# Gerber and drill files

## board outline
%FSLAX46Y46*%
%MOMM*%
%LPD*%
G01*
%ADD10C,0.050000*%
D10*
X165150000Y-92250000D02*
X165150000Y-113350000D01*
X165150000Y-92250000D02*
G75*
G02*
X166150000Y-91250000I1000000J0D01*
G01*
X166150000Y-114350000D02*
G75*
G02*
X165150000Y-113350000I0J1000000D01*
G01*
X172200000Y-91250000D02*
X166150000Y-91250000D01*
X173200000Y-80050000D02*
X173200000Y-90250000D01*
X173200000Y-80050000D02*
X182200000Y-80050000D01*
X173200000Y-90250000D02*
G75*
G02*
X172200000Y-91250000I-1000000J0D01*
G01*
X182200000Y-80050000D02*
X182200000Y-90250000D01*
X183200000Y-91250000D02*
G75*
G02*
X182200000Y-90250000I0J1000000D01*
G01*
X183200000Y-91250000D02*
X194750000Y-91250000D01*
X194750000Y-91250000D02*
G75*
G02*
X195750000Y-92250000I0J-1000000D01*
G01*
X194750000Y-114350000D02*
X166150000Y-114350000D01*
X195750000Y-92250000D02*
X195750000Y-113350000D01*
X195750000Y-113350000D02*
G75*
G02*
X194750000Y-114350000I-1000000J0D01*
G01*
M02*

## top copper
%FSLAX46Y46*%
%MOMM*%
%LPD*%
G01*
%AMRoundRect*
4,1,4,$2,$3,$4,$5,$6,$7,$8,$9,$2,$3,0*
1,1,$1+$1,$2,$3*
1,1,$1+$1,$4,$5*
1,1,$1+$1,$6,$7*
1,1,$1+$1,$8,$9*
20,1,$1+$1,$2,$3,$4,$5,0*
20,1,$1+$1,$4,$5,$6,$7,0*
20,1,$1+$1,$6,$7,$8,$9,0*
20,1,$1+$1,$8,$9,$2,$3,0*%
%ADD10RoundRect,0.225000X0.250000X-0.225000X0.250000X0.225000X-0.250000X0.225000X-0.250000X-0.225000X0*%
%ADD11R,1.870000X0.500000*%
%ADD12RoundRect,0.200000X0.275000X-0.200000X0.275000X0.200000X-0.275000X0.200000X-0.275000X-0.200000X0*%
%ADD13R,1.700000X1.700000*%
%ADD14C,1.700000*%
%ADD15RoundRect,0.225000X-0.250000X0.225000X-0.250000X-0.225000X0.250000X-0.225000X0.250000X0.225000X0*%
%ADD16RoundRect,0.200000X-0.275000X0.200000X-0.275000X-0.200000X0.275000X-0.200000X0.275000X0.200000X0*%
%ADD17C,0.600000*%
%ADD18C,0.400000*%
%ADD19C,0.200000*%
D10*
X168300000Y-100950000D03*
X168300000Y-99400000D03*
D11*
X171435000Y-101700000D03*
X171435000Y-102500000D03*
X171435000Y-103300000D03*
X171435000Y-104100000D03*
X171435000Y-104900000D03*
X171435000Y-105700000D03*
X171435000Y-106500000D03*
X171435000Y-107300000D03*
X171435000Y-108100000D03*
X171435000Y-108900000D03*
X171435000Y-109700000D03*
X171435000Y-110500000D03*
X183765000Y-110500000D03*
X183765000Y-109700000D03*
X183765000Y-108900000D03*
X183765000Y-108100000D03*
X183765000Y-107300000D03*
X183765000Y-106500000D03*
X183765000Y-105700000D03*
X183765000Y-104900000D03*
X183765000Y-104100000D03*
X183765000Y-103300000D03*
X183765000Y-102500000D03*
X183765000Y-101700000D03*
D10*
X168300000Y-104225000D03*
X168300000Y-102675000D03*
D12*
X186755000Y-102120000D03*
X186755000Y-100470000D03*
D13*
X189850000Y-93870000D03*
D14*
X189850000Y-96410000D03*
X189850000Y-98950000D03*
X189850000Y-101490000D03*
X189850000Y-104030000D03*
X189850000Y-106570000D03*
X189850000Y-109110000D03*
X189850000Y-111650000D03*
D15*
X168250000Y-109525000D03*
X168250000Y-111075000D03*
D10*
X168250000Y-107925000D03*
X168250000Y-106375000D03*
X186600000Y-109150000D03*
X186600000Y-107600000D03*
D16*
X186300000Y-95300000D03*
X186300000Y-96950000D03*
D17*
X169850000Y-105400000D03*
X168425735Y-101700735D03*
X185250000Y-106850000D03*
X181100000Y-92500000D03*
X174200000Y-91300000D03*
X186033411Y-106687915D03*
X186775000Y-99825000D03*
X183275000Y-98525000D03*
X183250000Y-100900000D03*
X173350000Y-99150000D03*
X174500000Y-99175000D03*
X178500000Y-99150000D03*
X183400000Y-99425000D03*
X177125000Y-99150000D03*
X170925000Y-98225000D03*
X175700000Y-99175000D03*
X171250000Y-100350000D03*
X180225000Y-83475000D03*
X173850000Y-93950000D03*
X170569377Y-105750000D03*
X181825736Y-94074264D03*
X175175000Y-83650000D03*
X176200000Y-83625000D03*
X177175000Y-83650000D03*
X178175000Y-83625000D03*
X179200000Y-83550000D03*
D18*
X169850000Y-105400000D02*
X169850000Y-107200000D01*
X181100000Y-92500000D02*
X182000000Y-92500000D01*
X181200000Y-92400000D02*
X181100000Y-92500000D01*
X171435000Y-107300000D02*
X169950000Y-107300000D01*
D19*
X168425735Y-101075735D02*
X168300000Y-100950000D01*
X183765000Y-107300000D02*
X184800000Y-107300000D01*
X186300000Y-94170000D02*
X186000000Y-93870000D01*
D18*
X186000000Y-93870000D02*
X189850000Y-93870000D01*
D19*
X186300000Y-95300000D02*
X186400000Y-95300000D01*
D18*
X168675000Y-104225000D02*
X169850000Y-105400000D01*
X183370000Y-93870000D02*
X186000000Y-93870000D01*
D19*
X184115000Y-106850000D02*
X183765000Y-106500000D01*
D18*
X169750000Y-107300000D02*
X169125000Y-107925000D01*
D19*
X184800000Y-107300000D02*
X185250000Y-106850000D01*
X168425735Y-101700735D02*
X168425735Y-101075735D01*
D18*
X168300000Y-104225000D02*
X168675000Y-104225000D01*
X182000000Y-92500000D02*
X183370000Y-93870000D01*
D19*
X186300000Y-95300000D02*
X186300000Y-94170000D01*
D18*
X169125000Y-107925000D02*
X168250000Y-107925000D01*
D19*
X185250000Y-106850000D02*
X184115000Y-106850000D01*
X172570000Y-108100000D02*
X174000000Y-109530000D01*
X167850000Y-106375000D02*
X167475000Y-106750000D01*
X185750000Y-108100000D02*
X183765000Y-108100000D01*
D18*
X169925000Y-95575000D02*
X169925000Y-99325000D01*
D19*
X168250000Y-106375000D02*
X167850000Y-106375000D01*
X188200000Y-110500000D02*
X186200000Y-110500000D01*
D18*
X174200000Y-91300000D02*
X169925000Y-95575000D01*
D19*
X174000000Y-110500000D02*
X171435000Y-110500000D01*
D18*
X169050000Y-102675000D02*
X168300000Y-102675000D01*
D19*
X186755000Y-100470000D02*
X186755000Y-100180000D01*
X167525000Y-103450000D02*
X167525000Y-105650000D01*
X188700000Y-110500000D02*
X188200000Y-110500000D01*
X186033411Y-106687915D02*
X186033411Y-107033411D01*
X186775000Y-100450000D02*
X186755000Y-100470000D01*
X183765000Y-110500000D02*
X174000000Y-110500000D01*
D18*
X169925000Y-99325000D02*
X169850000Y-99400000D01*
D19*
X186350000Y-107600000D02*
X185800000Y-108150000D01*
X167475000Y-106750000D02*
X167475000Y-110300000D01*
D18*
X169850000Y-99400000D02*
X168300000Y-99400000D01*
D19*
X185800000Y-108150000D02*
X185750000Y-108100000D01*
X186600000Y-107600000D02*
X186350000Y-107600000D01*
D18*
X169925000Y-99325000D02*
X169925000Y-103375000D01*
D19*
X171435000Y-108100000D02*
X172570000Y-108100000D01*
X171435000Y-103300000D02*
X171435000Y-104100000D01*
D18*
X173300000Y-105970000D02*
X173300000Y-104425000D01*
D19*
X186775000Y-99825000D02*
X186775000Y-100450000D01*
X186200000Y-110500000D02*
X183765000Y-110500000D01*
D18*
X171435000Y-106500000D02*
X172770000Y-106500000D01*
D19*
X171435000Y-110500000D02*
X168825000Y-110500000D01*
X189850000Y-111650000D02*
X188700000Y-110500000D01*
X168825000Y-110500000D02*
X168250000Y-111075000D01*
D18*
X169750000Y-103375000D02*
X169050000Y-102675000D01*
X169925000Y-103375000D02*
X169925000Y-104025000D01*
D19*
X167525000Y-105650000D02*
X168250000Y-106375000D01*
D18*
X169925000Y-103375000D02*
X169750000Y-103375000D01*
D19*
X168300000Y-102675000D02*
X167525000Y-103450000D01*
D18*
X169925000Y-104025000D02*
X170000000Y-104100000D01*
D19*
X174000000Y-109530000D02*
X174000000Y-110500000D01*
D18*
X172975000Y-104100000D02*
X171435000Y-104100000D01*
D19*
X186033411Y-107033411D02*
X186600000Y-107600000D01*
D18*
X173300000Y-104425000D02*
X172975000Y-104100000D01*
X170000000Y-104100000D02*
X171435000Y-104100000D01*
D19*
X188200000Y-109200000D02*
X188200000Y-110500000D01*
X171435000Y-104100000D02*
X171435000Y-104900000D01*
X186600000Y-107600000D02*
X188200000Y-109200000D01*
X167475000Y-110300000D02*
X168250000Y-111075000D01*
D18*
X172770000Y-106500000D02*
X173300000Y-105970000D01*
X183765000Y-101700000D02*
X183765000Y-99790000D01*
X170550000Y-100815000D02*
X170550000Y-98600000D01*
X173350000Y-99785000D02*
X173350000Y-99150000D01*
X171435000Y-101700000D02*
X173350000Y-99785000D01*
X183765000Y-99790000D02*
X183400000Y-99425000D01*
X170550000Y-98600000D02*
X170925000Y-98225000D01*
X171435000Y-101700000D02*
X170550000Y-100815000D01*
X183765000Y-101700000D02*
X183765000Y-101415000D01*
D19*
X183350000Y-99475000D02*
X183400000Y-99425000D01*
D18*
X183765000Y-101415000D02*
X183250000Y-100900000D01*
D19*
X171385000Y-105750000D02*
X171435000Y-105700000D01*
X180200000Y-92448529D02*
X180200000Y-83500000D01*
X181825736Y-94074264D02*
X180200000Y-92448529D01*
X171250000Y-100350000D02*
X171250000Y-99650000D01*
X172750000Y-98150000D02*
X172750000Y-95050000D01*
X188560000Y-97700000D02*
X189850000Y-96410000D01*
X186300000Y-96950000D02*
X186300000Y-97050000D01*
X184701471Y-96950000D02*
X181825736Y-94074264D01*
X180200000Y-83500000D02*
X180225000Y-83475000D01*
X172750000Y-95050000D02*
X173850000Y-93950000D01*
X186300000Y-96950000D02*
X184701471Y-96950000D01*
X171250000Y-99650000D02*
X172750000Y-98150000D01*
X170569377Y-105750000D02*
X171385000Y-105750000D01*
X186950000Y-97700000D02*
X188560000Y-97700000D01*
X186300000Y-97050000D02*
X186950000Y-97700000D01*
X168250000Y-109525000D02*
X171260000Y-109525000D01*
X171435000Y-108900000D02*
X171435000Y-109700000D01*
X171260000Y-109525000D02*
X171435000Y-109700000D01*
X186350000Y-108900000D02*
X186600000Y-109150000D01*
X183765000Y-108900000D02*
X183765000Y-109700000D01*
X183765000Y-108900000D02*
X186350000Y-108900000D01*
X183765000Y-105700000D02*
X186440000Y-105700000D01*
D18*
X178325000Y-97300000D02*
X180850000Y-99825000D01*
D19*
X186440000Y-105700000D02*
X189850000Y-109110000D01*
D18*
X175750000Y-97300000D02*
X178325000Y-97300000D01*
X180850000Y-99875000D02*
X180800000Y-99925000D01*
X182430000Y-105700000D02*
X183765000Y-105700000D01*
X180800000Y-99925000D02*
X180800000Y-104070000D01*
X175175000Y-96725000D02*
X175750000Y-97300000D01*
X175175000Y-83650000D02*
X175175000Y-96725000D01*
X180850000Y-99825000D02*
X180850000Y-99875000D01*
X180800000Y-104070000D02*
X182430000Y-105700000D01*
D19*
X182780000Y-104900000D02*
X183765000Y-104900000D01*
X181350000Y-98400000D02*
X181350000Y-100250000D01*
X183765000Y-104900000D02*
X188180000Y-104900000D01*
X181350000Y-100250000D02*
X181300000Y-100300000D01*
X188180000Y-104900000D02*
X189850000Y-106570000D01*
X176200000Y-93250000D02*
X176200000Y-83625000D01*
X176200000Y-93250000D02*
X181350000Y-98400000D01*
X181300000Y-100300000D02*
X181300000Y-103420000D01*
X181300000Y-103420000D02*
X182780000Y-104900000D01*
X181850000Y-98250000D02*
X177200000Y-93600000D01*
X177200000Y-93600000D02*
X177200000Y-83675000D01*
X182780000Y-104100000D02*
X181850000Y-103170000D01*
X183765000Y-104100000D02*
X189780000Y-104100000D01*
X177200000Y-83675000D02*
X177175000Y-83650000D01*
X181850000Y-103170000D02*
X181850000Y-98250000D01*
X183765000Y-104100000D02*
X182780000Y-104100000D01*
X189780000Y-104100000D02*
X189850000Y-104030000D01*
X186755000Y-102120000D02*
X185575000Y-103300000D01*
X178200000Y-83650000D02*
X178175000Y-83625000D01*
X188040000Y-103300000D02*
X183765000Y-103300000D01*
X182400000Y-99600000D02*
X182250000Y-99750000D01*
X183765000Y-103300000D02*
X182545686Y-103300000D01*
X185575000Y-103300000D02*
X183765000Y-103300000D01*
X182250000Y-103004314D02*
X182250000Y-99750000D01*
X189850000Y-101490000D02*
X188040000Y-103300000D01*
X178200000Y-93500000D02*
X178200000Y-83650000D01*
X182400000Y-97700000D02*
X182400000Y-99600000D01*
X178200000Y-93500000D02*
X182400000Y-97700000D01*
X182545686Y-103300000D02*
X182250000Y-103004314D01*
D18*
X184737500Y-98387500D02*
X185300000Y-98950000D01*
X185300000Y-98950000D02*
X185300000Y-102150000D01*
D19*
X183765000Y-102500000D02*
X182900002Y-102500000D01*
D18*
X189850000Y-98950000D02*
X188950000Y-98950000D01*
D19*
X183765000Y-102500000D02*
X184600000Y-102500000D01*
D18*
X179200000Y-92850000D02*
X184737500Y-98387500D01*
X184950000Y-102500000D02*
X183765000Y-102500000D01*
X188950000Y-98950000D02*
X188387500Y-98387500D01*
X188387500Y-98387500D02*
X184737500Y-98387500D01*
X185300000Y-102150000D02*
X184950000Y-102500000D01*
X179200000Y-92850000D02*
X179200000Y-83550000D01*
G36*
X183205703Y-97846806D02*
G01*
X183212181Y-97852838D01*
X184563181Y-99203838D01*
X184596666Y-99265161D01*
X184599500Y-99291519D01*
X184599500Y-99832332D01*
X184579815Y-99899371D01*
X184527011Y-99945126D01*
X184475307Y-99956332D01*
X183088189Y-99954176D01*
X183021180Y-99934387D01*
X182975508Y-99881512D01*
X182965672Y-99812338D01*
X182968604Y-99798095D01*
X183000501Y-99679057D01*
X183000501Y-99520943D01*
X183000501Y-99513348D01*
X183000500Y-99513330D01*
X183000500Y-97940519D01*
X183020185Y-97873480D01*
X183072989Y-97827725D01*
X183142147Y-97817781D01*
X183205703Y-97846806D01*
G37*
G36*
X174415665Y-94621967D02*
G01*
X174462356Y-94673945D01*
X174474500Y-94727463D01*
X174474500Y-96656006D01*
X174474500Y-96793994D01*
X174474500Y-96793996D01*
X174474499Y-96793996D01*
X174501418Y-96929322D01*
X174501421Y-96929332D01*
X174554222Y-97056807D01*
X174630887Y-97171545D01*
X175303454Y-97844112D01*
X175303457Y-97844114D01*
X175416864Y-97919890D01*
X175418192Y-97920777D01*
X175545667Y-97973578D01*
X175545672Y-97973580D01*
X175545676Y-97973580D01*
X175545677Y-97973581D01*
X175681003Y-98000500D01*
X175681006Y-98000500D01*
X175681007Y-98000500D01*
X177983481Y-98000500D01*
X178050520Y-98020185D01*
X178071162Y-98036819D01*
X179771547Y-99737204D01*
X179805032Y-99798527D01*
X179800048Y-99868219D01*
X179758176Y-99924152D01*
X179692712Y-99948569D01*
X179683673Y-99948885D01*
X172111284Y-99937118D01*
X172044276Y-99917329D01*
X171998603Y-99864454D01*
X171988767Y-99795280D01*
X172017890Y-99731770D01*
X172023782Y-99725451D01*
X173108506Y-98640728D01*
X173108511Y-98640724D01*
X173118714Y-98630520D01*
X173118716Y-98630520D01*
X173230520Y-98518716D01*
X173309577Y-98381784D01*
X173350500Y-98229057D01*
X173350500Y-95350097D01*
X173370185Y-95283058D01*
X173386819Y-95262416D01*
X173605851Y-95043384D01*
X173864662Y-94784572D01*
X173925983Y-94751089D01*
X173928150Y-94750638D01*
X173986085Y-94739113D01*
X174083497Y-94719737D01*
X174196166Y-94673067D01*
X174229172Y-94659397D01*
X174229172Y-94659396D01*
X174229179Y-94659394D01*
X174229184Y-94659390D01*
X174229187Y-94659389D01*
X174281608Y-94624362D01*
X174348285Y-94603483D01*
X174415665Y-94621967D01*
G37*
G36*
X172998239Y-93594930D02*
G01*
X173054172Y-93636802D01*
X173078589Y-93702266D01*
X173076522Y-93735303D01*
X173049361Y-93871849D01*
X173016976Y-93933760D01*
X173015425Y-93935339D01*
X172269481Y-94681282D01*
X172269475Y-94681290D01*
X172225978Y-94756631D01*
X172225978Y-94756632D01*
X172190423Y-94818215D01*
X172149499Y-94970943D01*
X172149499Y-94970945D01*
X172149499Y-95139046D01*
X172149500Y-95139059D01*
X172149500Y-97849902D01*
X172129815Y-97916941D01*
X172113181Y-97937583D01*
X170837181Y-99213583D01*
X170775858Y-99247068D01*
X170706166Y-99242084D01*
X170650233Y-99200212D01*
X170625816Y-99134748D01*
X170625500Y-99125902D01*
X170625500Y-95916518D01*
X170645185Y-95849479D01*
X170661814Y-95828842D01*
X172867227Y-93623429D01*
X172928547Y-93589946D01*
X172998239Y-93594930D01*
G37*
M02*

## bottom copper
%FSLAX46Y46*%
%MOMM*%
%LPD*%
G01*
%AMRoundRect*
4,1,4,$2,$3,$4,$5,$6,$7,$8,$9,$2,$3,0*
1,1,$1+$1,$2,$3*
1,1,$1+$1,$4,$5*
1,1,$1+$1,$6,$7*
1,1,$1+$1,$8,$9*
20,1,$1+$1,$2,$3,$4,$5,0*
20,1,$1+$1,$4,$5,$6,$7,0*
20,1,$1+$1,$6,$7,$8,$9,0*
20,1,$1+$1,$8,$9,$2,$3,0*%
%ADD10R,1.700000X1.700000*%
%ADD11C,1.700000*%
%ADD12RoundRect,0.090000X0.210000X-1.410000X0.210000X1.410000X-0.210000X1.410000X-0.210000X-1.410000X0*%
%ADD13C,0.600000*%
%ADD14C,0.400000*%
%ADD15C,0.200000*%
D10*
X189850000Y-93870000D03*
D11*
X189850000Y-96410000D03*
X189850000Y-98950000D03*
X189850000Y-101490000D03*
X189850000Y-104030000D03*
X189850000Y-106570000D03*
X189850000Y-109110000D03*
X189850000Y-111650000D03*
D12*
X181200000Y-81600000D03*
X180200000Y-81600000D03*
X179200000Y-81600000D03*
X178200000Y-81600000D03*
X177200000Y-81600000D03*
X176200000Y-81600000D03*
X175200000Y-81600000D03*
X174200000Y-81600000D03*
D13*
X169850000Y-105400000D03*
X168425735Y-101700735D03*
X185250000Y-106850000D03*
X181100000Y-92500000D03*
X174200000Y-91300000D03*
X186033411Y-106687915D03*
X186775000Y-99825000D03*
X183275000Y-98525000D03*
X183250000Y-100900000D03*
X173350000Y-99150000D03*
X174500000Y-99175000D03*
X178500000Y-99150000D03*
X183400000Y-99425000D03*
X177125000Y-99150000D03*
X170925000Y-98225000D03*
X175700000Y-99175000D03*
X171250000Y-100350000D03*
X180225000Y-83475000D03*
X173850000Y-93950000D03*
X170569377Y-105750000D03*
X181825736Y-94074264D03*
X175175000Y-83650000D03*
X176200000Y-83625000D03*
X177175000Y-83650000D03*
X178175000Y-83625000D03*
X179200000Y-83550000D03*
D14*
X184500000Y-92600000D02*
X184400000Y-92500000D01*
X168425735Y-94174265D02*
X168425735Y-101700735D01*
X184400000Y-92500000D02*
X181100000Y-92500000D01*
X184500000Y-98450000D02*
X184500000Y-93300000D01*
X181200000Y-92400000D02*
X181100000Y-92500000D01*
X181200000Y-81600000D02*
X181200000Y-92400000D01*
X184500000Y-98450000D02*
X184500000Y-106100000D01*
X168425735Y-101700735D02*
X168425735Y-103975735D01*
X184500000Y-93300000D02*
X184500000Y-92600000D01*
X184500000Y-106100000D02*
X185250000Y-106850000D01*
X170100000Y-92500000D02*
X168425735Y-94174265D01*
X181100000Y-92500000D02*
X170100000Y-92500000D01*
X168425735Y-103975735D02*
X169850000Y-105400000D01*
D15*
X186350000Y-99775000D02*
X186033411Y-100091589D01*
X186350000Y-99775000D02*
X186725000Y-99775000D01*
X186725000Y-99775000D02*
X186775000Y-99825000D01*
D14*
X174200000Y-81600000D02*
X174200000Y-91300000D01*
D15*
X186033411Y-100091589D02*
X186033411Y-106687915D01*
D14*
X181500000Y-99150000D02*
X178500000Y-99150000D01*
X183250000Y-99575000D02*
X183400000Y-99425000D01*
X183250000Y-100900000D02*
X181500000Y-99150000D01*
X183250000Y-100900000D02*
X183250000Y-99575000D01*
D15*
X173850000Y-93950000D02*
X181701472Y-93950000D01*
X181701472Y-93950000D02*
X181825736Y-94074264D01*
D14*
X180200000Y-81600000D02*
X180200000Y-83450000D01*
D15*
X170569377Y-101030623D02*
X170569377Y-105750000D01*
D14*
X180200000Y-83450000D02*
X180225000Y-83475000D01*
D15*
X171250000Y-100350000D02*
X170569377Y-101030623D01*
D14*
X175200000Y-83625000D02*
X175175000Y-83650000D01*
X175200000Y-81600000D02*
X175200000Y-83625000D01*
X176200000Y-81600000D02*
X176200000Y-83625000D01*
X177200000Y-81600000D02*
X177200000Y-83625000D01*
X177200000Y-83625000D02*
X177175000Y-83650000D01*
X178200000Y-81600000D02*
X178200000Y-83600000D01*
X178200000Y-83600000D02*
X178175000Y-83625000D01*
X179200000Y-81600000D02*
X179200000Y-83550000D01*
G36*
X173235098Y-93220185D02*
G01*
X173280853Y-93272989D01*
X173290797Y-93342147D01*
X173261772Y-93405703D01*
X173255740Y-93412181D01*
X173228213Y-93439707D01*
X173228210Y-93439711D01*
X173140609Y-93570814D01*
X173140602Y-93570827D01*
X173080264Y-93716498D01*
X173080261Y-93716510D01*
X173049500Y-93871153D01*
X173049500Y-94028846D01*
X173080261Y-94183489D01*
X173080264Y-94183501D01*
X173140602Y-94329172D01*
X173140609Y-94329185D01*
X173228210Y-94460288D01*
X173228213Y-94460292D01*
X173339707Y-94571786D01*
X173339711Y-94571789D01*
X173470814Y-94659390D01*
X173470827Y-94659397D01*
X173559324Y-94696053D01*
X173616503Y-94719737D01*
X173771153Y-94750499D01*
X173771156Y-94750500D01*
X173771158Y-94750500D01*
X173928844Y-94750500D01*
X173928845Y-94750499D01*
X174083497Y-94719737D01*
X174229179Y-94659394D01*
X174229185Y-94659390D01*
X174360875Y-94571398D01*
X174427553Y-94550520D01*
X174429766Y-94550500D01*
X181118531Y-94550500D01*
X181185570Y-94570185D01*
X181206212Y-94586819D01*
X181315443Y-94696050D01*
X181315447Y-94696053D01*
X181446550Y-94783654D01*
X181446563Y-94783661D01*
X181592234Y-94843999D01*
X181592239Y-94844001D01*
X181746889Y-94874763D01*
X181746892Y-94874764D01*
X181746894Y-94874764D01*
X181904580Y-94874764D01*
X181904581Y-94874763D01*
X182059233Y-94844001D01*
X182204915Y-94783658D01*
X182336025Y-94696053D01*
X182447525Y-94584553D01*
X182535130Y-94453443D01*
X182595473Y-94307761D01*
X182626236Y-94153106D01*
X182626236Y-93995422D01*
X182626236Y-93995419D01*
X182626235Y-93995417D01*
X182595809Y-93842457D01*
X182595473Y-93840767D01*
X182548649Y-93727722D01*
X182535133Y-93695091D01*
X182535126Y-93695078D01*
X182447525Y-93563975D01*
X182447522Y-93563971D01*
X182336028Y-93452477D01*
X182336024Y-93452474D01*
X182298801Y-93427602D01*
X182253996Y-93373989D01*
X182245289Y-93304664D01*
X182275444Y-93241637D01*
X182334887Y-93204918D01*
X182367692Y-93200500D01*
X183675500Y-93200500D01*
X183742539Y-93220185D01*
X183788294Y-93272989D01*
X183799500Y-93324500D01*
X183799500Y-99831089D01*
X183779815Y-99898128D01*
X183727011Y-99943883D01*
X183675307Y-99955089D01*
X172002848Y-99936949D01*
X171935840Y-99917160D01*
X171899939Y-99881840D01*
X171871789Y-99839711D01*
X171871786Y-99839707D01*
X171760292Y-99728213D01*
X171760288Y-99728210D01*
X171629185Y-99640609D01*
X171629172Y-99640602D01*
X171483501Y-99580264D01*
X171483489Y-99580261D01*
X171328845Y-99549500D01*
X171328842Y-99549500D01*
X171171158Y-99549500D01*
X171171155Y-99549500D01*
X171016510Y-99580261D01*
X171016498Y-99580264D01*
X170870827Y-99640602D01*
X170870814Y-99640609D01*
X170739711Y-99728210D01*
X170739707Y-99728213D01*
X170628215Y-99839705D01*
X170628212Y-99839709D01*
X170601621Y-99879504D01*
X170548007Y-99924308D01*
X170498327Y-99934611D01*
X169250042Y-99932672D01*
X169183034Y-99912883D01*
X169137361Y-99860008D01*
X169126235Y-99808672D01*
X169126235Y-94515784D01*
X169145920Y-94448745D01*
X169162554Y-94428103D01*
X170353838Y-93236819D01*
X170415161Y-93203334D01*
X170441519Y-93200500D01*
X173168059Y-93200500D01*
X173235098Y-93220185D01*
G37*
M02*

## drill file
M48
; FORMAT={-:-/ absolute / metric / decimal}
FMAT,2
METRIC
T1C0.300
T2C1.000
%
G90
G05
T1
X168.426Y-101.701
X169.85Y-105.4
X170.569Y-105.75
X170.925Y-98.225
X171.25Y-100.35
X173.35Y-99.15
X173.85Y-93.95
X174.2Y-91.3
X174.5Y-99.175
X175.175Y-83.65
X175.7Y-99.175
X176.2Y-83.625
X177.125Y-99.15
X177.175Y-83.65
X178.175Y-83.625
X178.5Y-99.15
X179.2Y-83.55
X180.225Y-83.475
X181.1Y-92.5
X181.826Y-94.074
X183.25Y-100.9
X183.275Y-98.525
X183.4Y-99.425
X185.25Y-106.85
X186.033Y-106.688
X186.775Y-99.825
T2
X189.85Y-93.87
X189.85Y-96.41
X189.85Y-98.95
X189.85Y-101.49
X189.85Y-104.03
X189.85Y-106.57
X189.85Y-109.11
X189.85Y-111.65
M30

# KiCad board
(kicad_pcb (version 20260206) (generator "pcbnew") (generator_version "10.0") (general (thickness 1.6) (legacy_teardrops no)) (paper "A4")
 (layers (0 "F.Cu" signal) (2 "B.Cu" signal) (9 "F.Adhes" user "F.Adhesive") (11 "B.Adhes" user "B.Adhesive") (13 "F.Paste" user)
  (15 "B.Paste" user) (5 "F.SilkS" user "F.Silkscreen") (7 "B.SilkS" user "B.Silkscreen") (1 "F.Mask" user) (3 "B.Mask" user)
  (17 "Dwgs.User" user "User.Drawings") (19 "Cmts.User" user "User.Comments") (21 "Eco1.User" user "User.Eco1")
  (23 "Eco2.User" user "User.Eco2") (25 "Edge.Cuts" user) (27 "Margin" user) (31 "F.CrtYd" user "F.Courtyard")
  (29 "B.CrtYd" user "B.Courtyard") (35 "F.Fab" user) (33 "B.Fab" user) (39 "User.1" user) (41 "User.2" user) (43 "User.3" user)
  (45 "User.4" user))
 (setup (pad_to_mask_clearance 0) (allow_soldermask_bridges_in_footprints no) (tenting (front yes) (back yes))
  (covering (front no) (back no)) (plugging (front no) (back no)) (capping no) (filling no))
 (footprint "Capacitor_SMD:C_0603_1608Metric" (layer "F.Cu") (at 168.3 100.175 90)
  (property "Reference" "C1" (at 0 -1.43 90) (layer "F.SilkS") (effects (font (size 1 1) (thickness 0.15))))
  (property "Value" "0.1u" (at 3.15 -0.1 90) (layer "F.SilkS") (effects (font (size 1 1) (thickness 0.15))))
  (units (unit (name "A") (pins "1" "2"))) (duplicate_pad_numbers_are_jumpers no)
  (pad "1" smd roundrect (at -0.775 0 90) (size 0.9 0.95) (layers "F.Cu" "F.Mask" "F.Paste") (roundrect_rratio 0.25) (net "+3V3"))
  (pad "2" smd roundrect (at 0.775 0 90) (size 0.9 0.95) (layers "F.Cu" "F.Mask" "F.Paste") (roundrect_rratio 0.25) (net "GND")))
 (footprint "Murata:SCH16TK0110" (layer "F.Cu") (at 177.6 106.1)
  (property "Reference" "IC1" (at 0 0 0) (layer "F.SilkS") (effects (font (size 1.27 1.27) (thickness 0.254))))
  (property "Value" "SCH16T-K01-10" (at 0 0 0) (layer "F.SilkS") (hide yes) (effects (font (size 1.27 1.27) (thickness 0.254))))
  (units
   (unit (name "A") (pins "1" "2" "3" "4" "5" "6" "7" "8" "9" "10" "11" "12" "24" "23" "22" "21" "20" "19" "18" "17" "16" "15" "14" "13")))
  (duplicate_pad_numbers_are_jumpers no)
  (pad "1" smd rect (at -6.165 -4.4 90) (size 0.5 1.87) (layers "F.Cu" "F.Mask" "F.Paste") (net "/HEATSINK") (thermal_bridge_angle 45))
  (pad "2" smd rect (at -6.165 -3.6 90) (size 0.5 1.87) (layers "F.Cu" "F.Mask" "F.Paste") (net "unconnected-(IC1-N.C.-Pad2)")
   (thermal_bridge_angle 45))
  (pad "3" smd rect (at -6.165 -2.8 90) (size 0.5 1.87) (layers "F.Cu" "F.Mask" "F.Paste") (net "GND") (thermal_bridge_angle 45))
  (pad "4" smd rect (at -6.165 -2 90) (size 0.5 1.87) (layers "F.Cu" "F.Mask" "F.Paste") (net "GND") (thermal_bridge_angle 45))
  (pad "5" smd rect (at -6.165 -1.2 90) (size 0.5 1.87) (layers "F.Cu" "F.Mask" "F.Paste") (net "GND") (thermal_bridge_angle 45))
  (pad "6" smd rect (at -6.165 -0.4 90) (size 0.5 1.87) (layers "F.Cu" "F.Mask" "F.Paste") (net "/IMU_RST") (thermal_bridge_angle 45))
  (pad "7" smd rect (at -6.165 0.4 90) (size 0.5 1.87) (layers "F.Cu" "F.Mask" "F.Paste") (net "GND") (thermal_bridge_angle 45))
  (pad "8" smd rect (at -6.165 1.2 90) (size 0.5 1.87) (layers "F.Cu" "F.Mask" "F.Paste") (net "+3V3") (thermal_bridge_angle 45))
  (pad "9" smd rect (at -6.165 2 90) (size 0.5 1.87) (layers "F.Cu" "F.Mask" "F.Paste") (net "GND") (thermal_bridge_angle 45))
  (pad "10" smd rect (at -6.165 2.8 90) (size 0.5 1.87) (layers "F.Cu" "F.Mask" "F.Paste") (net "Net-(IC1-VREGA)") (thermal_bridge_angle 45))
  (pad "11" smd rect (at -6.165 3.6 90) (size 0.5 1.87) (layers "F.Cu" "F.Mask" "F.Paste") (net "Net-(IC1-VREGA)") (thermal_bridge_angle 45))
  (pad "12" smd rect (at -6.165 4.4 90) (size 0.5 1.87) (layers "F.Cu" "F.Mask" "F.Paste") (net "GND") (thermal_bridge_angle 45))
  (pad "13" smd rect (at 6.165 4.4 90) (size 0.5 1.87) (layers "F.Cu" "F.Mask" "F.Paste") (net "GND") (thermal_bridge_angle 45))
  (pad "14" smd rect (at 6.165 3.6 90) (size 0.5 1.87) (layers "F.Cu" "F.Mask" "F.Paste") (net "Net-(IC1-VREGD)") (thermal_bridge_angle 45))
  (pad "15" smd rect (at 6.165 2.8 90) (size 0.5 1.87) (layers "F.Cu" "F.Mask" "F.Paste") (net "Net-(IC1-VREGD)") (thermal_bridge_angle 45))
  (pad "16" smd rect (at 6.165 2 90) (size 0.5 1.87) (layers "F.Cu" "F.Mask" "F.Paste") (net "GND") (thermal_bridge_angle 45))
  (pad "17" smd rect (at 6.165 1.2 90) (size 0.5 1.87) (layers "F.Cu" "F.Mask" "F.Paste") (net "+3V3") (thermal_bridge_angle 45))
  (pad "18" smd rect (at 6.165 0.4 90) (size 0.5 1.87) (layers "F.Cu" "F.Mask" "F.Paste") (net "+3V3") (thermal_bridge_angle 45))
  (pad "19" smd rect (at 6.165 -0.4 90) (size 0.5 1.87) (layers "F.Cu" "F.Mask" "F.Paste") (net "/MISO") (thermal_bridge_angle 45))
  (pad "20" smd rect (at 6.165 -1.2 90) (size 0.5 1.87) (layers "F.Cu" "F.Mask" "F.Paste") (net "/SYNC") (thermal_bridge_angle 45))
  (pad "21" smd rect (at 6.165 -2 90) (size 0.5 1.87) (layers "F.Cu" "F.Mask" "F.Paste") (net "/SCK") (thermal_bridge_angle 45))
  (pad "22" smd rect (at 6.165 -2.8 90) (size 0.5 1.87) (layers "F.Cu" "F.Mask" "F.Paste") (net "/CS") (thermal_bridge_angle 45))
  (pad "23" smd rect (at 6.165 -3.6 90) (size 0.5 1.87) (layers "F.Cu" "F.Mask" "F.Paste") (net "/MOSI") (thermal_bridge_angle 45))
  (pad "24" smd rect (at 6.165 -4.4 90) (size 0.5 1.87) (layers "F.Cu" "F.Mask" "F.Paste") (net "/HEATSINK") (thermal_bridge_angle 45)))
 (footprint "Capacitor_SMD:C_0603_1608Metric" (layer "F.Cu") (at 168.3 103.45 90)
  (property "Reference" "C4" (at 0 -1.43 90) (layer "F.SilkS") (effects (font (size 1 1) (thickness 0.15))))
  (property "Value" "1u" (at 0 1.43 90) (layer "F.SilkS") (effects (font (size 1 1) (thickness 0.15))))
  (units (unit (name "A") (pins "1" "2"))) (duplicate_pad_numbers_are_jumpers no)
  (pad "1" smd roundrect (at -0.775 0 90) (size 0.9 0.95) (layers "F.Cu" "F.Mask" "F.Paste") (roundrect_rratio 0.25) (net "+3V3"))
  (pad "2" smd roundrect (at 0.775 0 90) (size 0.9 0.95) (layers "F.Cu" "F.Mask" "F.Paste") (roundrect_rratio 0.25) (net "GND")))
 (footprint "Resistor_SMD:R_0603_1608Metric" (layer "F.Cu") (at 186.755 101.295 90)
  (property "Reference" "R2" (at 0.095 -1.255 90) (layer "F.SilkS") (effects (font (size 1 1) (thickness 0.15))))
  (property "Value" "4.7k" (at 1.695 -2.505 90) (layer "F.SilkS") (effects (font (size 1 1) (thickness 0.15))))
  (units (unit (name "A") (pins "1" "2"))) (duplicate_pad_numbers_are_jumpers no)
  (pad "1" smd roundrect (at -0.825 0 90) (size 0.8 0.95) (layers "F.Cu" "F.Mask" "F.Paste") (roundrect_rratio 0.25) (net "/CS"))
  (pad "2" smd roundrect (at 0.825 0 90) (size 0.8 0.95) (layers "F.Cu" "F.Mask" "F.Paste") (roundrect_rratio 0.25) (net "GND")))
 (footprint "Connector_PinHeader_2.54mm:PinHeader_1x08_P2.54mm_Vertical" (layer "F.Cu") (at 189.85 93.87)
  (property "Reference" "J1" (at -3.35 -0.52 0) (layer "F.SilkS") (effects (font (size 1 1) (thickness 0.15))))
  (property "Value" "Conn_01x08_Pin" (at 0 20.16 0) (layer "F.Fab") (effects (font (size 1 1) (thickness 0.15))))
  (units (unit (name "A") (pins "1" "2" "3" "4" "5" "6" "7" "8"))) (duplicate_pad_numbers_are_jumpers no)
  (pad "1" thru_hole rect (at 0 0) (size 1.7 1.7) (drill 1) (layers "*.Cu" "*.Mask") (remove_unused_layers no) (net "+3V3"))
  (pad "2" thru_hole circle (at 0 2.54) (size 1.7 1.7) (drill 1) (layers "*.Cu" "*.Mask") (remove_unused_layers no) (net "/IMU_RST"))
  (pad "3" thru_hole circle (at 0 5.08) (size 1.7 1.7) (drill 1) (layers "*.Cu" "*.Mask") (remove_unused_layers no) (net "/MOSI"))
  (pad "4" thru_hole circle (at 0 7.62) (size 1.7 1.7) (drill 1) (layers "*.Cu" "*.Mask") (remove_unused_layers no) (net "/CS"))
  (pad "5" thru_hole circle (at 0 10.16) (size 1.7 1.7) (drill 1) (layers "*.Cu" "*.Mask") (remove_unused_layers no) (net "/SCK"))
  (pad "6" thru_hole circle (at 0 12.7) (size 1.7 1.7) (drill 1) (layers "*.Cu" "*.Mask") (remove_unused_layers no) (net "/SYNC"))
  (pad "7" thru_hole circle (at 0 15.24) (size 1.7 1.7) (drill 1) (layers "*.Cu" "*.Mask") (remove_unused_layers no) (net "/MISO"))
  (pad "8" thru_hole circle (at 0 17.78) (size 1.7 1.7) (drill 1) (layers "*.Cu" "*.Mask") (remove_unused_layers no) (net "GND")))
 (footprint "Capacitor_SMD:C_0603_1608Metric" (layer "F.Cu") (at 168.25 110.3 -90)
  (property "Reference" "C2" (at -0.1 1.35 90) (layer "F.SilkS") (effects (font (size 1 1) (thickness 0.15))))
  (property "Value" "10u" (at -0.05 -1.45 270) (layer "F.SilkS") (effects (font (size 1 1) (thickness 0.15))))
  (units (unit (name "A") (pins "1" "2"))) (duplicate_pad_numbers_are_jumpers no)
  (pad "1" smd roundrect (at -0.775 0 270) (size 0.9 0.95) (layers "F.Cu" "F.Mask" "F.Paste") (roundrect_rratio 0.25)
   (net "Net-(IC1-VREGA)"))
  (pad "2" smd roundrect (at 0.775 0 270) (size 0.9 0.95) (layers "F.Cu" "F.Mask" "F.Paste") (roundrect_rratio 0.25) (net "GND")))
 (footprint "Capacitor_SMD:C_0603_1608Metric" (layer "F.Cu") (at 168.25 107.15 90)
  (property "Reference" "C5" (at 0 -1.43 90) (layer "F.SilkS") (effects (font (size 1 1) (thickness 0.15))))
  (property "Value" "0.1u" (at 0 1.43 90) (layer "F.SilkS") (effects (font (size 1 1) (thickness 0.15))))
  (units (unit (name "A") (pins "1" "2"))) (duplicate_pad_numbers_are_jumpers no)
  (pad "1" smd roundrect (at -0.775 0 90) (size 0.9 0.95) (layers "F.Cu" "F.Mask" "F.Paste") (roundrect_rratio 0.25) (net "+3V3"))
  (pad "2" smd roundrect (at 0.775 0 90) (size 0.9 0.95) (layers "F.Cu" "F.Mask" "F.Paste") (roundrect_rratio 0.25) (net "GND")))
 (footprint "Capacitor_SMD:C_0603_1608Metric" (layer "F.Cu") (at 186.6 108.375 90)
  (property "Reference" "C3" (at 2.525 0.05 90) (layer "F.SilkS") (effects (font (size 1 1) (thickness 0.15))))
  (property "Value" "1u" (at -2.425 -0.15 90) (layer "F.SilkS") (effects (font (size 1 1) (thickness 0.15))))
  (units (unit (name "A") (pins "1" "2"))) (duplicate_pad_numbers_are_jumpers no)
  (pad "1" smd roundrect (at -0.775 0 90) (size 0.9 0.95) (layers "F.Cu" "F.Mask" "F.Paste") (roundrect_rratio 0.25) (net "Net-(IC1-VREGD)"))
  (pad "2" smd roundrect (at 0.775 0 90) (size 0.9 0.95) (layers "F.Cu" "F.Mask" "F.Paste") (roundrect_rratio 0.25) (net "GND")))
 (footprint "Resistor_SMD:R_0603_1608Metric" (layer "F.Cu") (at 186.3 96.125 -90)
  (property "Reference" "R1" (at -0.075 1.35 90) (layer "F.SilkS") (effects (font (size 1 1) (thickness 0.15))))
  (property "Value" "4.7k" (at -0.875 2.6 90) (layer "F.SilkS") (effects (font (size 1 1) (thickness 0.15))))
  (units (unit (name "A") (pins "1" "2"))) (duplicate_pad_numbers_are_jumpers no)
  (pad "1" smd roundrect (at -0.825 0 270) (size 0.8 0.95) (layers "F.Cu" "F.Mask" "F.Paste") (roundrect_rratio 0.25) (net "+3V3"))
  (pad "2" smd roundrect (at 0.825 0 270) (size 0.8 0.95) (layers "F.Cu" "F.Mask" "F.Paste") (roundrect_rratio 0.25) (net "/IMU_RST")))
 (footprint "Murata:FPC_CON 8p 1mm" (layer "B.Cu") (at 177.7 81.6 90)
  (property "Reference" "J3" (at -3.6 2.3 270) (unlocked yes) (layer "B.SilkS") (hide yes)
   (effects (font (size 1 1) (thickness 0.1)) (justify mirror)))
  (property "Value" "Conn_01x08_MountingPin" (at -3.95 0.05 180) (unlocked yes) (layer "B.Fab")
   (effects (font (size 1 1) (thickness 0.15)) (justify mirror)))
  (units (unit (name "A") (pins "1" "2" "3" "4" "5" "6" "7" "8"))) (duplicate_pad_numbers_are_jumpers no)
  (pad "1" smd roundrect (at 0 3.5 90) (size 3 0.6) (layers "B.Cu" "B.Mask" "B.Paste") (roundrect_rratio 0.15) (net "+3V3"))
  (pad "2" smd roundrect (at 0 2.5 90) (size 3 0.6) (layers "B.Cu" "B.Mask" "B.Paste") (roundrect_rratio 0.15) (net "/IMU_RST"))
  (pad "3" smd roundrect (at 0 1.5 90) (size 3 0.6) (layers "B.Cu" "B.Mask" "B.Paste") (roundrect_rratio 0.15) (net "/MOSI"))
  (pad "4" smd roundrect (at 0 0.5 90) (size 3 0.6) (layers "B.Cu" "B.Mask" "B.Paste") (roundrect_rratio 0.15) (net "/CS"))
  (pad "5" smd roundrect (at 0 -0.5 90) (size 3 0.6) (layers "B.Cu" "B.Mask" "B.Paste") (roundrect_rratio 0.15) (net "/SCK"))
  (pad "6" smd roundrect (at 0 -1.5 90) (size 3 0.6) (layers "B.Cu" "B.Mask" "B.Paste") (roundrect_rratio 0.15) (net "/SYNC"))
  (pad "7" smd roundrect (at 0 -2.5 90) (size 3 0.6) (layers "B.Cu" "B.Mask" "B.Paste") (roundrect_rratio 0.15) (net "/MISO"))
  (pad "8" smd roundrect (at 0 -3.5 90) (size 3 0.6) (layers "B.Cu" "B.Mask" "B.Paste") (roundrect_rratio 0.15) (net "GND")))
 (gr_line (start 165.15 92.25) (end 165.15 113.35) (stroke (width 0.05) (type default)) (layer "Edge.Cuts"))
 (gr_arc (start 165.15 92.25) (mid 165.442893 91.542893) (end 166.15 91.25) (stroke (width 0.05) (type default)) (layer "Edge.Cuts"))
 (gr_arc (start 166.15 114.35) (mid 165.442893 114.057107) (end 165.15 113.35) (stroke (width 0.05) (type default)) (layer "Edge.Cuts"))
 (gr_line (start 172.2 91.25) (end 166.15 91.25) (stroke (width 0.05) (type default)) (layer "Edge.Cuts"))
 (gr_line (start 173.2 80.05) (end 173.2 90.25) (stroke (width 0.05) (type default)) (layer "Edge.Cuts"))
 (gr_line (start 173.2 80.05) (end 182.2 80.05) (stroke (width 0.05) (type default)) (layer "Edge.Cuts"))
 (gr_arc (start 173.2 90.25) (mid 172.907107 90.957107) (end 172.2 91.25) (stroke (width 0.05) (type default)) (layer "Edge.Cuts"))
 (gr_line (start 182.2 80.05) (end 182.2 90.25) (stroke (width 0.05) (type default)) (layer "Edge.Cuts"))
 (gr_arc (start 183.2 91.25) (mid 182.492893 90.957107) (end 182.2 90.25) (stroke (width 0.05) (type default)) (layer "Edge.Cuts"))
 (gr_line (start 183.2 91.25) (end 194.75 91.25) (stroke (width 0.05) (type default)) (layer "Edge.Cuts"))
 (gr_arc (start 194.75 91.25) (mid 195.457107 91.542893) (end 195.75 92.25) (stroke (width 0.05) (type default)) (layer "Edge.Cuts"))
 (gr_line (start 194.75 114.35) (end 166.15 114.35) (stroke (width 0.05) (type default)) (layer "Edge.Cuts"))
 (gr_line (start 195.75 92.25) (end 195.75 113.35) (stroke (width 0.05) (type default)) (layer "Edge.Cuts"))
 (gr_arc (start 195.75 113.35) (mid 195.457107 114.057107) (end 194.75 114.35) (stroke (width 0.05) (type default)) (layer "Edge.Cuts"))
 (segment (start 169.85 105.4) (end 169.85 107.2) (width 0.4) (layer "F.Cu") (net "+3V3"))
 (segment (start 181.1 92.5) (end 182 92.5) (width 0.4) (layer "F.Cu") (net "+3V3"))
 (segment (start 181.2 92.4) (end 181.1 92.5) (width 0.4) (layer "F.Cu") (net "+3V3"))
 (segment (start 171.435 107.3) (end 169.95 107.3) (width 0.4) (layer "F.Cu") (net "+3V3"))
 (segment (start 168.425735 101.075735) (end 168.3 100.95) (width 0.2) (layer "F.Cu") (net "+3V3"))
 (segment (start 183.765 107.3) (end 184.8 107.3) (width 0.2) (layer "F.Cu") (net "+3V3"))
 (segment (start 186.3 94.17) (end 186 93.87) (width 0.2) (layer "F.Cu") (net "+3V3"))
 (segment (start 186 93.87) (end 189.85 93.87) (width 0.4) (layer "F.Cu") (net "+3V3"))
 (segment (start 186.3 95.3) (end 186.4 95.3) (width 0.2) (layer "F.Cu") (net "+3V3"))
 (segment (start 168.675 104.225) (end 169.85 105.4) (width 0.4) (layer "F.Cu") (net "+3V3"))
 (segment (start 183.37 93.87) (end 186 93.87) (width 0.4) (layer "F.Cu") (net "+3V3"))
 (segment (start 184.115 106.85) (end 183.765 106.5) (width 0.2) (layer "F.Cu") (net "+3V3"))
 (segment (start 169.75 107.3) (end 169.125 107.925) (width 0.4) (layer "F.Cu") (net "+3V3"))
 (segment (start 184.8 107.3) (end 185.25 106.85) (width 0.2) (layer "F.Cu") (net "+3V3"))
 (segment (start 168.425735 101.700735) (end 168.425735 101.075735) (width 0.2) (layer "F.Cu") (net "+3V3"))
 (segment (start 168.3 104.225) (end 168.675 104.225) (width 0.4) (layer "F.Cu") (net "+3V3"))
 (segment (start 182 92.5) (end 183.37 93.87) (width 0.4) (layer "F.Cu") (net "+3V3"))
 (segment (start 186.3 95.3) (end 186.3 94.17) (width 0.2) (layer "F.Cu") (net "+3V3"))
 (segment (start 169.125 107.925) (end 168.25 107.925) (width 0.4) (layer "F.Cu") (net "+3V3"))
 (segment (start 185.25 106.85) (end 184.115 106.85) (width 0.2) (layer "F.Cu") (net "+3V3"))
 (via (at 169.85 105.4) (size 0.6) (drill 0.3) (layers "F.Cu" "B.Cu") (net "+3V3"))
 (via (at 168.425735 101.700735) (size 0.6) (drill 0.3) (layers "F.Cu" "B.Cu") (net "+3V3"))
 (via (at 185.25 106.85) (size 0.6) (drill 0.3) (layers "F.Cu" "B.Cu") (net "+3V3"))
 (via (at 181.1 92.5) (size 0.6) (drill 0.3) (layers "F.Cu" "B.Cu") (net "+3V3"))
 (segment (start 184.5 92.6) (end 184.4 92.5) (width 0.4) (layer "B.Cu") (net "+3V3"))
 (segment (start 168.425735 94.174265) (end 168.425735 101.700735) (width 0.4) (layer "B.Cu") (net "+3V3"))
 (segment (start 184.4 92.5) (end 181.1 92.5) (width 0.4) (layer "B.Cu") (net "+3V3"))
 (segment (start 184.5 98.45) (end 184.5 93.3) (width 0.4) (layer "B.Cu") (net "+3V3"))
 (segment (start 181.2 92.4) (end 181.1 92.5) (width 0.4) (layer "B.Cu") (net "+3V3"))
 (segment (start 181.2 81.6) (end 181.2 92.4) (width 0.4) (layer "B.Cu") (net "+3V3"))
 (segment (start 184.5 98.45) (end 184.5 106.1) (width 0.4) (layer "B.Cu") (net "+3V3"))
 (segment (start 168.425735 101.700735) (end 168.425735 103.975735) (width 0.4) (layer "B.Cu") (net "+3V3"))
 (segment (start 184.5 93.3) (end 184.5 92.6) (width 0.4) (layer "B.Cu") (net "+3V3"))
 (segment (start 184.5 106.1) (end 185.25 106.85) (width 0.4) (layer "B.Cu") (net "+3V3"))
 (segment (start 170.1 92.5) (end 168.425735 94.174265) (width 0.4) (layer "B.Cu") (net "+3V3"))
 (segment (start 181.1 92.5) (end 170.1 92.5) (width 0.4) (layer "B.Cu") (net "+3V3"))
 (segment (start 168.425735 103.975735) (end 169.85 105.4) (width 0.4) (layer "B.Cu") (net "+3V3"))
 (segment (start 172.57 108.1) (end 174 109.53) (width 0.2) (layer "F.Cu") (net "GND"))
 (segment (start 167.85 106.375) (end 167.475 106.75) (width 0.2) (layer "F.Cu") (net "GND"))
 (segment (start 185.75 108.1) (end 183.765 108.1) (width 0.2) (layer "F.Cu") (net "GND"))
 (segment (start 169.925 95.575) (end 169.925 99.325) (width 0.4) (layer "F.Cu") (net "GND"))
 (segment (start 168.25 106.375) (end 167.85 106.375) (width 0.2) (layer "F.Cu") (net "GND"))
 (segment (start 188.2 110.5) (end 186.2 110.5) (width 0.2) (layer "F.Cu") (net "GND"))
 (segment (start 174.2 91.3) (end 169.925 95.575) (width 0.4) (layer "F.Cu") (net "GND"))
 (segment (start 174 110.5) (end 171.435 110.5) (width 0.2) (layer "F.Cu") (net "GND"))
 (segment (start 169.05 102.675) (end 168.3 102.675) (width 0.4) (layer "F.Cu") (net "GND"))
 (segment (start 186.755 100.47) (end 186.755 100.18) (width 0.2) (layer "F.Cu") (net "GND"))
 (segment (start 167.525 103.45) (end 167.525 105.65) (width 0.2) (layer "F.Cu") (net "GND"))
 (segment (start 188.7 110.5) (end 188.2 110.5) (width 0.2) (layer "F.Cu") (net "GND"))
 (segment (start 186.033411 106.687915) (end 186.033411 107.033411) (width 0.2) (layer "F.Cu") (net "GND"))
 (segment (start 186.775 100.45) (end 186.755 100.47) (width 0.2) (layer "F.Cu") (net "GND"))
 (segment (start 183.765 110.5) (end 174 110.5) (width 0.2) (layer "F.Cu") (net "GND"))
 (segment (start 169.925 99.325) (end 169.85 99.4) (width 0.4) (layer "F.Cu") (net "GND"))
 (segment (start 186.35 107.6) (end 185.8 108.15) (width 0.2) (layer "F.Cu") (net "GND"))
 (segment (start 167.475 106.75) (end 167.475 110.3) (width 0.2) (layer "F.Cu") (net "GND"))
 (segment (start 169.85 99.4) (end 168.3 99.4) (width 0.4) (layer "F.Cu") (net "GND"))
 (segment (start 185.8 108.15) (end 185.75 108.1) (width 0.2) (layer "F.Cu") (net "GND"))
 (segment (start 186.6 107.6) (end 186.35 107.6) (width 0.2) (layer "F.Cu") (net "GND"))
 (segment (start 169.925 99.325) (end 169.925 103.375) (width 0.4) (layer "F.Cu") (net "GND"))
 (segment (start 171.435 108.1) (end 172.57 108.1) (width 0.2) (layer "F.Cu") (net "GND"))
 (segment (start 171.435 103.3) (end 171.435 104.1) (width 0.2) (layer "F.Cu") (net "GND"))
 (segment (start 173.3 105.97) (end 173.3 104.425) (width 0.4) (layer "F.Cu") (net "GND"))
 (segment (start 186.775 99.825) (end 186.775 100.45) (width 0.2) (layer "F.Cu") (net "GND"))
 (segment (start 186.2 110.5) (end 183.765 110.5) (width 0.2) (layer "F.Cu") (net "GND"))
 (segment (start 171.435 106.5) (end 172.77 106.5) (width 0.4) (layer "F.Cu") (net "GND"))
 (segment (start 171.435 110.5) (end 168.825 110.5) (width 0.2) (layer "F.Cu") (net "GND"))
 (segment (start 189.85 111.65) (end 188.7 110.5) (width 0.2) (layer "F.Cu") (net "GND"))
 (segment (start 168.825 110.5) (end 168.25 111.075) (width 0.2) (layer "F.Cu") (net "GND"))
 (segment (start 169.75 103.375) (end 169.05 102.675) (width 0.4) (layer "F.Cu") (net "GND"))
 (segment (start 169.925 103.375) (end 169.925 104.025) (width 0.4) (layer "F.Cu") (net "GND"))
 (segment (start 167.525 105.65) (end 168.25 106.375) (width 0.2) (layer "F.Cu") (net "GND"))
 (segment (start 169.925 103.375) (end 169.75 103.375) (width 0.4) (layer "F.Cu") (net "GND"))
 (segment (start 168.3 102.675) (end 167.525 103.45) (width 0.2) (layer "F.Cu") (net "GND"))
 (segment (start 169.925 104.025) (end 170 104.1) (width 0.4) (layer "F.Cu") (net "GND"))
 (segment (start 174 109.53) (end 174 110.5) (width 0.2) (layer "F.Cu") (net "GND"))
 (segment (start 172.975 104.1) (end 171.435 104.1) (width 0.4) (layer "F.Cu") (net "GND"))
 (segment (start 186.033411 107.033411) (end 186.6 107.6) (width 0.2) (layer "F.Cu") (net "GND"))
 (segment (start 173.3 104.425) (end 172.975 104.1) (width 0.4) (layer "F.Cu") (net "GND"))
 (segment (start 170 104.1) (end 171.435 104.1) (width 0.4) (layer "F.Cu") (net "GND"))
 (segment (start 188.2 109.2) (end 188.2 110.5) (width 0.2) (layer "F.Cu") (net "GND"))
 (segment (start 171.435 104.1) (end 171.435 104.9) (width 0.2) (layer "F.Cu") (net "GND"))
 (segment (start 186.6 107.6) (end 188.2 109.2) (width 0.2) (layer "F.Cu") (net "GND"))
 (segment (start 167.475 110.3) (end 168.25 111.075) (width 0.2) (layer "F.Cu") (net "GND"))
 (segment (start 172.77 106.5) (end 173.3 105.97) (width 0.4) (layer "F.Cu") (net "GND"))
 (via (at 174.2 91.3) (size 0.6) (drill 0.3) (layers "F.Cu" "B.Cu") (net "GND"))
 (via (at 186.033411 106.687915) (size 0.6) (drill 0.3) (layers "F.Cu" "B.Cu") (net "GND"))
 (via (at 186.775 99.825) (size 0.6) (drill 0.3) (layers "F.Cu" "B.Cu") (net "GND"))
 (segment (start 186.35 99.775) (end 186.033411 100.091589) (width 0.2) (layer "B.Cu") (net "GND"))
 (segment (start 186.35 99.775) (end 186.725 99.775) (width 0.2) (layer "B.Cu") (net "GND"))
 (segment (start 186.725 99.775) (end 186.775 99.825) (width 0.2) (layer "B.Cu") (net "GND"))
 (segment (start 174.2 81.6) (end 174.2 91.3) (width 0.4) (layer "B.Cu") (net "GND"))
 (segment (start 186.033411 100.091589) (end 186.033411 106.687915) (width 0.2) (layer "B.Cu") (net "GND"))
 (segment (start 183.765 101.7) (end 183.765 99.79) (width 0.4) (layer "F.Cu") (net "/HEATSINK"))
 (segment (start 170.55 100.815) (end 170.55 98.6) (width 0.4) (layer "F.Cu") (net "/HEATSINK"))
 (segment (start 173.35 99.785) (end 173.35 99.15) (width 0.4) (layer "F.Cu") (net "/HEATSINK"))
 (segment (start 171.435 101.7) (end 173.35 99.785) (width 0.4) (layer "F.Cu") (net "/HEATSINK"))
 (segment (start 183.765 99.79) (end 183.4 99.425) (width 0.4) (layer "F.Cu") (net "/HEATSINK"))
 (segment (start 170.55 98.6) (end 170.925 98.225) (width 0.4) (layer "F.Cu") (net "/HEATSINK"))
 (segment (start 171.435 101.7) (end 170.55 100.815) (width 0.4) (layer "F.Cu") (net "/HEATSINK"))
 (segment (start 183.765 101.7) (end 183.765 101.415) (width 0.4) (layer "F.Cu") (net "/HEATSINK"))
 (segment (start 183.35 99.475) (end 183.4 99.425) (width 0.2) (layer "F.Cu") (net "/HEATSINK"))
 (segment (start 183.765 101.415) (end 183.25 100.9) (width 0.4) (layer "F.Cu") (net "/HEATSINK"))
 (via (at 183.275 98.525) (size 0.6) (drill 0.3) (layers "F.Cu" "B.Cu") (free yes) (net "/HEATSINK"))
 (via (at 183.25 100.9) (size 0.6) (drill 0.3) (layers "F.Cu" "B.Cu") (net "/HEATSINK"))
 (via (at 173.35 99.15) (size 0.6) (drill 0.3) (layers "F.Cu" "B.Cu") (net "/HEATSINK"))
 (via (at 174.5 99.175) (size 0.6) (drill 0.3) (layers "F.Cu" "B.Cu") (free yes) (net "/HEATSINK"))
 (via (at 178.5 99.15) (size 0.6) (drill 0.3) (layers "F.Cu" "B.Cu") (free yes) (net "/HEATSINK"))
 (via (at 183.4 99.425) (size 0.6) (drill 0.3) (layers "F.Cu" "B.Cu") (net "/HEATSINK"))
 (via (at 177.125 99.15) (size 0.6) (drill 0.3) (layers "F.Cu" "B.Cu") (free yes) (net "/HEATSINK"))
 (via (at 170.925 98.225) (size 0.6) (drill 0.3) (layers "F.Cu" "B.Cu") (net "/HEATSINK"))
 (via (at 175.7 99.175) (size 0.6) (drill 0.3) (layers "F.Cu" "B.Cu") (free yes) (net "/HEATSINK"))
 (segment (start 181.5 99.15) (end 178.5 99.15) (width 0.4) (layer "B.Cu") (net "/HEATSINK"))
 (segment (start 183.25 99.575) (end 183.4 99.425) (width 0.4) (layer "B.Cu") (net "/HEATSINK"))
 (segment (start 183.25 100.9) (end 181.5 99.15) (width 0.4) (layer "B.Cu") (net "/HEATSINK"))
 (segment (start 183.25 100.9) (end 183.25 99.575) (width 0.4) (layer "B.Cu") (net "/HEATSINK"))
 (segment (start 171.385 105.75) (end 171.435 105.7) (width 0.2) (layer "F.Cu") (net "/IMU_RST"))
 (segment (start 180.2 92.448529) (end 180.2 83.5) (width 0.2) (layer "F.Cu") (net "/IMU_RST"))
 (segment (start 181.825736 94.074264) (end 180.2 92.448529) (width 0.2) (layer "F.Cu") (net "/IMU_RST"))
 (segment (start 171.25 100.35) (end 171.25 99.65) (width 0.2) (layer "F.Cu") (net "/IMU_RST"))
 (segment (start 172.75 98.15) (end 172.75 95.05) (width 0.2) (layer "F.Cu") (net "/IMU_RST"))
 (segment (start 188.56 97.7) (end 189.85 96.41) (width 0.2) (layer "F.Cu") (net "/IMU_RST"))
 (segment (start 186.3 96.95) (end 186.3 97.05) (width 0.2) (layer "F.Cu") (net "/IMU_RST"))
 (segment (start 184.701471 96.95) (end 181.825736 94.074264) (width 0.2) (layer "F.Cu") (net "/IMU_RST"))
 (segment (start 180.2 83.5) (end 180.225 83.475) (width 0.2) (layer "F.Cu") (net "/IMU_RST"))
 (segment (start 172.75 95.05) (end 173.85 93.95) (width 0.2) (layer "F.Cu") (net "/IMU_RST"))
 (segment (start 186.3 96.95) (end 184.701471 96.95) (width 0.2) (layer "F.Cu") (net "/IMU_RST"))
 (segment (start 171.25 99.65) (end 172.75 98.15) (width 0.2) (layer "F.Cu") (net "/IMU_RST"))
 (segment (start 170.569377 105.75) (end 171.385 105.75) (width 0.2) (layer "F.Cu") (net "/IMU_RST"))
 (segment (start 186.95 97.7) (end 188.56 97.7) (width 0.2) (layer "F.Cu") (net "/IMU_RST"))
 (segment (start 186.3 97.05) (end 186.95 97.7) (width 0.2) (layer "F.Cu") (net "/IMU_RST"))
 (via (at 171.25 100.35) (size 0.6) (drill 0.3) (layers "F.Cu" "B.Cu") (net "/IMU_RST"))
 (via (at 180.225 83.475) (size 0.6) (drill 0.3) (layers "F.Cu" "B.Cu") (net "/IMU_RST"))
 (via (at 173.85 93.95) (size 0.6) (drill 0.3) (layers "F.Cu" "B.Cu") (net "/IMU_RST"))
 (via (at 170.569377 105.75) (size 0.6) (drill 0.3) (layers "F.Cu" "B.Cu") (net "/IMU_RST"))
 (via (at 181.825736 94.074264) (size 0.6) (drill 0.3) (layers "F.Cu" "B.Cu") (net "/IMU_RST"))
 (segment (start 173.85 93.95) (end 181.701472 93.95) (width 0.2) (layer "B.Cu") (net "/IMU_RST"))
 (segment (start 181.701472 93.95) (end 181.825736 94.074264) (width 0.2) (layer "B.Cu") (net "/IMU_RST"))
 (segment (start 180.2 81.6) (end 180.2 83.45) (width 0.4) (layer "B.Cu") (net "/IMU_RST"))
 (segment (start 170.569377 101.030623) (end 170.569377 105.75) (width 0.2) (layer "B.Cu") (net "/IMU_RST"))
 (segment (start 180.2 83.45) (end 180.225 83.475) (width 0.4) (layer "B.Cu") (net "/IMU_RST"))
 (segment (start 171.25 100.35) (end 170.569377 101.030623) (width 0.2) (layer "B.Cu") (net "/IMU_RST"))
 (segment (start 168.25 109.525) (end 171.26 109.525) (width 0.2) (layer "F.Cu") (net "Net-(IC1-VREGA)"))
 (segment (start 171.435 108.9) (end 171.435 109.7) (width 0.2) (layer "F.Cu") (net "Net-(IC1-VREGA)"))
 (segment (start 171.26 109.525) (end 171.435 109.7) (width 0.2) (layer "F.Cu") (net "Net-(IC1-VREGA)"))
 (segment (start 186.35 108.9) (end 186.6 109.15) (width 0.2) (layer "F.Cu") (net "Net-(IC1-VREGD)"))
 (segment (start 183.765 108.9) (end 183.765 109.7) (width 0.2) (layer "F.Cu") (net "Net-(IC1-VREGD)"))
 (segment (start 183.765 108.9) (end 186.35 108.9) (width 0.2) (layer "F.Cu") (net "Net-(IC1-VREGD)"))
 (segment (start 183.765 105.7) (end 186.44 105.7) (width 0.2) (layer "F.Cu") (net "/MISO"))
 (segment (start 178.325 97.3) (end 180.85 99.825) (width 0.4) (layer "F.Cu") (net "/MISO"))
 (segment (start 186.44 105.7) (end 189.85 109.11) (width 0.2) (layer "F.Cu") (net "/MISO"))
 (segment (start 175.75 97.3) (end 178.325 97.3) (width 0.4) (layer "F.Cu") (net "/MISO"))
 (segment (start 180.85 99.875) (end 180.8 99.925) (width 0.4) (layer "F.Cu") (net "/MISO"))
 (segment (start 182.43 105.7) (end 183.765 105.7) (width 0.4) (layer "F.Cu") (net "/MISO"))
 (segment (start 180.8 99.925) (end 180.8 104.07) (width 0.4) (layer "F.Cu") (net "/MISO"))
 (segment (start 175.175 96.725) (end 175.75 97.3) (width 0.4) (layer "F.Cu") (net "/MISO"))
 (segment (start 175.175 83.65) (end 175.175 96.725) (width 0.4) (layer "F.Cu") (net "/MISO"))
 (segment (start 180.85 99.825) (end 180.85 99.875) (width 0.4) (layer "F.Cu") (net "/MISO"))
 (segment (start 180.8 104.07) (end 182.43 105.7) (width 0.4) (layer "F.Cu") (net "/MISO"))
 (via (at 175.175 83.65) (size 0.6) (drill 0.3) (layers "F.Cu" "B.Cu") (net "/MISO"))
 (segment (start 175.2 83.625) (end 175.175 83.65) (width 0.4) (layer "B.Cu") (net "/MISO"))
 (segment (start 175.2 81.6) (end 175.2 83.625) (width 0.4) (layer "B.Cu") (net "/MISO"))
 (segment (start 182.78 104.9) (end 183.765 104.9) (width 0.2) (layer "F.Cu") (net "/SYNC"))
 (segment (start 181.35 98.4) (end 181.35 100.25) (width 0.2) (layer "F.Cu") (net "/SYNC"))
 (segment (start 183.765 104.9) (end 188.18 104.9) (width 0.2) (layer "F.Cu") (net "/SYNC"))
 (segment (start 181.35 100.25) (end 181.3 100.3) (width 0.2) (layer "F.Cu") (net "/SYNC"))
 (segment (start 188.18 104.9) (end 189.85 106.57) (width 0.2) (layer "F.Cu") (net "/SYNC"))
 (segment (start 176.2 93.25) (end 176.2 83.625) (width 0.2) (layer "F.Cu") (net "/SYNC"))
 (segment (start 176.2 93.25) (end 181.35 98.4) (width 0.2) (layer "F.Cu") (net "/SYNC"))
 (segment (start 181.3 100.3) (end 181.3 103.42) (width 0.2) (layer "F.Cu") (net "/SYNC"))
 (segment (start 181.3 103.42) (end 182.78 104.9) (width 0.2) (layer "F.Cu") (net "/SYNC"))
 (via (at 176.2 83.625) (size 0.6) (drill 0.3) (layers "F.Cu" "B.Cu") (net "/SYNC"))
 (segment (start 176.2 81.6) (end 176.2 83.625) (width 0.4) (layer "B.Cu") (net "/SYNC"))
 (segment (start 181.85 98.25) (end 177.2 93.6) (width 0.2) (layer "F.Cu") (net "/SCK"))
 (segment (start 177.2 93.6) (end 177.2 83.675) (width 0.2) (layer "F.Cu") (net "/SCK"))
 (segment (start 182.78 104.1) (end 181.85 103.17) (width 0.2) (layer "F.Cu") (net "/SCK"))
 (segment (start 183.765 104.1) (end 189.78 104.1) (width 0.2) (layer "F.Cu") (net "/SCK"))
 (segment (start 177.2 83.675) (end 177.175 83.65) (width 0.2) (layer "F.Cu") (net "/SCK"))
 (segment (start 181.85 103.17) (end 181.85 98.25) (width 0.2) (layer "F.Cu") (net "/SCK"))
 (segment (start 183.765 104.1) (end 182.78 104.1) (width 0.2) (layer "F.Cu") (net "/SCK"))
 (segment (start 189.78 104.1) (end 189.85 104.03) (width 0.2) (layer "F.Cu") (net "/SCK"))
 (via (at 177.175 83.65) (size 0.6) (drill 0.3) (layers "F.Cu" "B.Cu") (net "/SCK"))
 (segment (start 177.2 81.6) (end 177.2 83.625) (width 0.4) (layer "B.Cu") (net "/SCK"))
 (segment (start 177.2 83.625) (end 177.175 83.65) (width 0.4) (layer "B.Cu") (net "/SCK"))
 (segment (start 186.755 102.12) (end 185.575 103.3) (width 0.2) (layer "F.Cu") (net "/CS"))
 (segment (start 178.2 83.65) (end 178.175 83.625) (width 0.2) (layer "F.Cu") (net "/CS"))
 (segment (start 188.04 103.3) (end 183.765 103.3) (width 0.2) (layer "F.Cu") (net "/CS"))
 (segment (start 182.4 99.6) (end 182.25 99.75) (width 0.2) (layer "F.Cu") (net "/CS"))
 (segment (start 183.765 103.3) (end 182.545686 103.3) (width 0.2) (layer "F.Cu") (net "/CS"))
 (segment (start 185.575 103.3) (end 183.765 103.3) (width 0.2) (layer "F.Cu") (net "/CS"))
 (segment (start 182.25 103.004314) (end 182.25 99.75) (width 0.2) (layer "F.Cu") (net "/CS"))
 (segment (start 189.85 101.49) (end 188.04 103.3) (width 0.2) (layer "F.Cu") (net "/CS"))
 (segment (start 178.2 93.5) (end 178.2 83.65) (width 0.2) (layer "F.Cu") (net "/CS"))
 (segment (start 182.4 97.7) (end 182.4 99.6) (width 0.2) (layer "F.Cu") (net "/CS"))
 (segment (start 178.2 93.5) (end 182.4 97.7) (width 0.2) (layer "F.Cu") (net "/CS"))
 (segment (start 182.545686 103.3) (end 182.25 103.004314) (width 0.2) (layer "F.Cu") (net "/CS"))
 (via (at 178.175 83.625) (size 0.6) (drill 0.3) (layers "F.Cu" "B.Cu") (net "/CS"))
 (segment (start 178.2 81.6) (end 178.2 83.6) (width 0.4) (layer "B.Cu") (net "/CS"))
 (segment (start 178.2 83.6) (end 178.175 83.625) (width 0.4) (layer "B.Cu") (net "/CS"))
 (segment (start 184.7375 98.3875) (end 185.3 98.95) (width 0.4) (layer "F.Cu") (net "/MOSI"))
 (segment (start 185.3 98.95) (end 185.3 102.15) (width 0.4) (layer "F.Cu") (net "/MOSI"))
 (segment (start 183.765 102.5) (end 182.900002 102.5) (width 0.2) (layer "F.Cu") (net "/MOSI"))
 (segment (start 189.85 98.95) (end 188.95 98.95) (width 0.4) (layer "F.Cu") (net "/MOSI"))
 (segment (start 183.765 102.5) (end 184.6 102.5) (width 0.2) (layer "F.Cu") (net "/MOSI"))
 (segment (start 179.2 92.85) (end 184.7375 98.3875) (width 0.4) (layer "F.Cu") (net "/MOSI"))
 (segment (start 184.95 102.5) (end 183.765 102.5) (width 0.4) (layer "F.Cu") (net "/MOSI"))
 (segment (start 188.95 98.95) (end 188.3875 98.3875) (width 0.4) (layer "F.Cu") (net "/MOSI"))
 (segment (start 188.3875 98.3875) (end 184.7375 98.3875) (width 0.4) (layer "F.Cu") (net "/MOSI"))
 (segment (start 185.3 102.15) (end 184.95 102.5) (width 0.4) (layer "F.Cu") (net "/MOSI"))
 (segment (start 179.2 92.85) (end 179.2 83.55) (width 0.4) (layer "F.Cu") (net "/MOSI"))
 (via (at 179.2 83.55) (size 0.6) (drill 0.3) (layers "F.Cu" "B.Cu") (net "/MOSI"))
 (segment (start 179.2 81.6) (end 179.2 83.55) (width 0.4) (layer "B.Cu") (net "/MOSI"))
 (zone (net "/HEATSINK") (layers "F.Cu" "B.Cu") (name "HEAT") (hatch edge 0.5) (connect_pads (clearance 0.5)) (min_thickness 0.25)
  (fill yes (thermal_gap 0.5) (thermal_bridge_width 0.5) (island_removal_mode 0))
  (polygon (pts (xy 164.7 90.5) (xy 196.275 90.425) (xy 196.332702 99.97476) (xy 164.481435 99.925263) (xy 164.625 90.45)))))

